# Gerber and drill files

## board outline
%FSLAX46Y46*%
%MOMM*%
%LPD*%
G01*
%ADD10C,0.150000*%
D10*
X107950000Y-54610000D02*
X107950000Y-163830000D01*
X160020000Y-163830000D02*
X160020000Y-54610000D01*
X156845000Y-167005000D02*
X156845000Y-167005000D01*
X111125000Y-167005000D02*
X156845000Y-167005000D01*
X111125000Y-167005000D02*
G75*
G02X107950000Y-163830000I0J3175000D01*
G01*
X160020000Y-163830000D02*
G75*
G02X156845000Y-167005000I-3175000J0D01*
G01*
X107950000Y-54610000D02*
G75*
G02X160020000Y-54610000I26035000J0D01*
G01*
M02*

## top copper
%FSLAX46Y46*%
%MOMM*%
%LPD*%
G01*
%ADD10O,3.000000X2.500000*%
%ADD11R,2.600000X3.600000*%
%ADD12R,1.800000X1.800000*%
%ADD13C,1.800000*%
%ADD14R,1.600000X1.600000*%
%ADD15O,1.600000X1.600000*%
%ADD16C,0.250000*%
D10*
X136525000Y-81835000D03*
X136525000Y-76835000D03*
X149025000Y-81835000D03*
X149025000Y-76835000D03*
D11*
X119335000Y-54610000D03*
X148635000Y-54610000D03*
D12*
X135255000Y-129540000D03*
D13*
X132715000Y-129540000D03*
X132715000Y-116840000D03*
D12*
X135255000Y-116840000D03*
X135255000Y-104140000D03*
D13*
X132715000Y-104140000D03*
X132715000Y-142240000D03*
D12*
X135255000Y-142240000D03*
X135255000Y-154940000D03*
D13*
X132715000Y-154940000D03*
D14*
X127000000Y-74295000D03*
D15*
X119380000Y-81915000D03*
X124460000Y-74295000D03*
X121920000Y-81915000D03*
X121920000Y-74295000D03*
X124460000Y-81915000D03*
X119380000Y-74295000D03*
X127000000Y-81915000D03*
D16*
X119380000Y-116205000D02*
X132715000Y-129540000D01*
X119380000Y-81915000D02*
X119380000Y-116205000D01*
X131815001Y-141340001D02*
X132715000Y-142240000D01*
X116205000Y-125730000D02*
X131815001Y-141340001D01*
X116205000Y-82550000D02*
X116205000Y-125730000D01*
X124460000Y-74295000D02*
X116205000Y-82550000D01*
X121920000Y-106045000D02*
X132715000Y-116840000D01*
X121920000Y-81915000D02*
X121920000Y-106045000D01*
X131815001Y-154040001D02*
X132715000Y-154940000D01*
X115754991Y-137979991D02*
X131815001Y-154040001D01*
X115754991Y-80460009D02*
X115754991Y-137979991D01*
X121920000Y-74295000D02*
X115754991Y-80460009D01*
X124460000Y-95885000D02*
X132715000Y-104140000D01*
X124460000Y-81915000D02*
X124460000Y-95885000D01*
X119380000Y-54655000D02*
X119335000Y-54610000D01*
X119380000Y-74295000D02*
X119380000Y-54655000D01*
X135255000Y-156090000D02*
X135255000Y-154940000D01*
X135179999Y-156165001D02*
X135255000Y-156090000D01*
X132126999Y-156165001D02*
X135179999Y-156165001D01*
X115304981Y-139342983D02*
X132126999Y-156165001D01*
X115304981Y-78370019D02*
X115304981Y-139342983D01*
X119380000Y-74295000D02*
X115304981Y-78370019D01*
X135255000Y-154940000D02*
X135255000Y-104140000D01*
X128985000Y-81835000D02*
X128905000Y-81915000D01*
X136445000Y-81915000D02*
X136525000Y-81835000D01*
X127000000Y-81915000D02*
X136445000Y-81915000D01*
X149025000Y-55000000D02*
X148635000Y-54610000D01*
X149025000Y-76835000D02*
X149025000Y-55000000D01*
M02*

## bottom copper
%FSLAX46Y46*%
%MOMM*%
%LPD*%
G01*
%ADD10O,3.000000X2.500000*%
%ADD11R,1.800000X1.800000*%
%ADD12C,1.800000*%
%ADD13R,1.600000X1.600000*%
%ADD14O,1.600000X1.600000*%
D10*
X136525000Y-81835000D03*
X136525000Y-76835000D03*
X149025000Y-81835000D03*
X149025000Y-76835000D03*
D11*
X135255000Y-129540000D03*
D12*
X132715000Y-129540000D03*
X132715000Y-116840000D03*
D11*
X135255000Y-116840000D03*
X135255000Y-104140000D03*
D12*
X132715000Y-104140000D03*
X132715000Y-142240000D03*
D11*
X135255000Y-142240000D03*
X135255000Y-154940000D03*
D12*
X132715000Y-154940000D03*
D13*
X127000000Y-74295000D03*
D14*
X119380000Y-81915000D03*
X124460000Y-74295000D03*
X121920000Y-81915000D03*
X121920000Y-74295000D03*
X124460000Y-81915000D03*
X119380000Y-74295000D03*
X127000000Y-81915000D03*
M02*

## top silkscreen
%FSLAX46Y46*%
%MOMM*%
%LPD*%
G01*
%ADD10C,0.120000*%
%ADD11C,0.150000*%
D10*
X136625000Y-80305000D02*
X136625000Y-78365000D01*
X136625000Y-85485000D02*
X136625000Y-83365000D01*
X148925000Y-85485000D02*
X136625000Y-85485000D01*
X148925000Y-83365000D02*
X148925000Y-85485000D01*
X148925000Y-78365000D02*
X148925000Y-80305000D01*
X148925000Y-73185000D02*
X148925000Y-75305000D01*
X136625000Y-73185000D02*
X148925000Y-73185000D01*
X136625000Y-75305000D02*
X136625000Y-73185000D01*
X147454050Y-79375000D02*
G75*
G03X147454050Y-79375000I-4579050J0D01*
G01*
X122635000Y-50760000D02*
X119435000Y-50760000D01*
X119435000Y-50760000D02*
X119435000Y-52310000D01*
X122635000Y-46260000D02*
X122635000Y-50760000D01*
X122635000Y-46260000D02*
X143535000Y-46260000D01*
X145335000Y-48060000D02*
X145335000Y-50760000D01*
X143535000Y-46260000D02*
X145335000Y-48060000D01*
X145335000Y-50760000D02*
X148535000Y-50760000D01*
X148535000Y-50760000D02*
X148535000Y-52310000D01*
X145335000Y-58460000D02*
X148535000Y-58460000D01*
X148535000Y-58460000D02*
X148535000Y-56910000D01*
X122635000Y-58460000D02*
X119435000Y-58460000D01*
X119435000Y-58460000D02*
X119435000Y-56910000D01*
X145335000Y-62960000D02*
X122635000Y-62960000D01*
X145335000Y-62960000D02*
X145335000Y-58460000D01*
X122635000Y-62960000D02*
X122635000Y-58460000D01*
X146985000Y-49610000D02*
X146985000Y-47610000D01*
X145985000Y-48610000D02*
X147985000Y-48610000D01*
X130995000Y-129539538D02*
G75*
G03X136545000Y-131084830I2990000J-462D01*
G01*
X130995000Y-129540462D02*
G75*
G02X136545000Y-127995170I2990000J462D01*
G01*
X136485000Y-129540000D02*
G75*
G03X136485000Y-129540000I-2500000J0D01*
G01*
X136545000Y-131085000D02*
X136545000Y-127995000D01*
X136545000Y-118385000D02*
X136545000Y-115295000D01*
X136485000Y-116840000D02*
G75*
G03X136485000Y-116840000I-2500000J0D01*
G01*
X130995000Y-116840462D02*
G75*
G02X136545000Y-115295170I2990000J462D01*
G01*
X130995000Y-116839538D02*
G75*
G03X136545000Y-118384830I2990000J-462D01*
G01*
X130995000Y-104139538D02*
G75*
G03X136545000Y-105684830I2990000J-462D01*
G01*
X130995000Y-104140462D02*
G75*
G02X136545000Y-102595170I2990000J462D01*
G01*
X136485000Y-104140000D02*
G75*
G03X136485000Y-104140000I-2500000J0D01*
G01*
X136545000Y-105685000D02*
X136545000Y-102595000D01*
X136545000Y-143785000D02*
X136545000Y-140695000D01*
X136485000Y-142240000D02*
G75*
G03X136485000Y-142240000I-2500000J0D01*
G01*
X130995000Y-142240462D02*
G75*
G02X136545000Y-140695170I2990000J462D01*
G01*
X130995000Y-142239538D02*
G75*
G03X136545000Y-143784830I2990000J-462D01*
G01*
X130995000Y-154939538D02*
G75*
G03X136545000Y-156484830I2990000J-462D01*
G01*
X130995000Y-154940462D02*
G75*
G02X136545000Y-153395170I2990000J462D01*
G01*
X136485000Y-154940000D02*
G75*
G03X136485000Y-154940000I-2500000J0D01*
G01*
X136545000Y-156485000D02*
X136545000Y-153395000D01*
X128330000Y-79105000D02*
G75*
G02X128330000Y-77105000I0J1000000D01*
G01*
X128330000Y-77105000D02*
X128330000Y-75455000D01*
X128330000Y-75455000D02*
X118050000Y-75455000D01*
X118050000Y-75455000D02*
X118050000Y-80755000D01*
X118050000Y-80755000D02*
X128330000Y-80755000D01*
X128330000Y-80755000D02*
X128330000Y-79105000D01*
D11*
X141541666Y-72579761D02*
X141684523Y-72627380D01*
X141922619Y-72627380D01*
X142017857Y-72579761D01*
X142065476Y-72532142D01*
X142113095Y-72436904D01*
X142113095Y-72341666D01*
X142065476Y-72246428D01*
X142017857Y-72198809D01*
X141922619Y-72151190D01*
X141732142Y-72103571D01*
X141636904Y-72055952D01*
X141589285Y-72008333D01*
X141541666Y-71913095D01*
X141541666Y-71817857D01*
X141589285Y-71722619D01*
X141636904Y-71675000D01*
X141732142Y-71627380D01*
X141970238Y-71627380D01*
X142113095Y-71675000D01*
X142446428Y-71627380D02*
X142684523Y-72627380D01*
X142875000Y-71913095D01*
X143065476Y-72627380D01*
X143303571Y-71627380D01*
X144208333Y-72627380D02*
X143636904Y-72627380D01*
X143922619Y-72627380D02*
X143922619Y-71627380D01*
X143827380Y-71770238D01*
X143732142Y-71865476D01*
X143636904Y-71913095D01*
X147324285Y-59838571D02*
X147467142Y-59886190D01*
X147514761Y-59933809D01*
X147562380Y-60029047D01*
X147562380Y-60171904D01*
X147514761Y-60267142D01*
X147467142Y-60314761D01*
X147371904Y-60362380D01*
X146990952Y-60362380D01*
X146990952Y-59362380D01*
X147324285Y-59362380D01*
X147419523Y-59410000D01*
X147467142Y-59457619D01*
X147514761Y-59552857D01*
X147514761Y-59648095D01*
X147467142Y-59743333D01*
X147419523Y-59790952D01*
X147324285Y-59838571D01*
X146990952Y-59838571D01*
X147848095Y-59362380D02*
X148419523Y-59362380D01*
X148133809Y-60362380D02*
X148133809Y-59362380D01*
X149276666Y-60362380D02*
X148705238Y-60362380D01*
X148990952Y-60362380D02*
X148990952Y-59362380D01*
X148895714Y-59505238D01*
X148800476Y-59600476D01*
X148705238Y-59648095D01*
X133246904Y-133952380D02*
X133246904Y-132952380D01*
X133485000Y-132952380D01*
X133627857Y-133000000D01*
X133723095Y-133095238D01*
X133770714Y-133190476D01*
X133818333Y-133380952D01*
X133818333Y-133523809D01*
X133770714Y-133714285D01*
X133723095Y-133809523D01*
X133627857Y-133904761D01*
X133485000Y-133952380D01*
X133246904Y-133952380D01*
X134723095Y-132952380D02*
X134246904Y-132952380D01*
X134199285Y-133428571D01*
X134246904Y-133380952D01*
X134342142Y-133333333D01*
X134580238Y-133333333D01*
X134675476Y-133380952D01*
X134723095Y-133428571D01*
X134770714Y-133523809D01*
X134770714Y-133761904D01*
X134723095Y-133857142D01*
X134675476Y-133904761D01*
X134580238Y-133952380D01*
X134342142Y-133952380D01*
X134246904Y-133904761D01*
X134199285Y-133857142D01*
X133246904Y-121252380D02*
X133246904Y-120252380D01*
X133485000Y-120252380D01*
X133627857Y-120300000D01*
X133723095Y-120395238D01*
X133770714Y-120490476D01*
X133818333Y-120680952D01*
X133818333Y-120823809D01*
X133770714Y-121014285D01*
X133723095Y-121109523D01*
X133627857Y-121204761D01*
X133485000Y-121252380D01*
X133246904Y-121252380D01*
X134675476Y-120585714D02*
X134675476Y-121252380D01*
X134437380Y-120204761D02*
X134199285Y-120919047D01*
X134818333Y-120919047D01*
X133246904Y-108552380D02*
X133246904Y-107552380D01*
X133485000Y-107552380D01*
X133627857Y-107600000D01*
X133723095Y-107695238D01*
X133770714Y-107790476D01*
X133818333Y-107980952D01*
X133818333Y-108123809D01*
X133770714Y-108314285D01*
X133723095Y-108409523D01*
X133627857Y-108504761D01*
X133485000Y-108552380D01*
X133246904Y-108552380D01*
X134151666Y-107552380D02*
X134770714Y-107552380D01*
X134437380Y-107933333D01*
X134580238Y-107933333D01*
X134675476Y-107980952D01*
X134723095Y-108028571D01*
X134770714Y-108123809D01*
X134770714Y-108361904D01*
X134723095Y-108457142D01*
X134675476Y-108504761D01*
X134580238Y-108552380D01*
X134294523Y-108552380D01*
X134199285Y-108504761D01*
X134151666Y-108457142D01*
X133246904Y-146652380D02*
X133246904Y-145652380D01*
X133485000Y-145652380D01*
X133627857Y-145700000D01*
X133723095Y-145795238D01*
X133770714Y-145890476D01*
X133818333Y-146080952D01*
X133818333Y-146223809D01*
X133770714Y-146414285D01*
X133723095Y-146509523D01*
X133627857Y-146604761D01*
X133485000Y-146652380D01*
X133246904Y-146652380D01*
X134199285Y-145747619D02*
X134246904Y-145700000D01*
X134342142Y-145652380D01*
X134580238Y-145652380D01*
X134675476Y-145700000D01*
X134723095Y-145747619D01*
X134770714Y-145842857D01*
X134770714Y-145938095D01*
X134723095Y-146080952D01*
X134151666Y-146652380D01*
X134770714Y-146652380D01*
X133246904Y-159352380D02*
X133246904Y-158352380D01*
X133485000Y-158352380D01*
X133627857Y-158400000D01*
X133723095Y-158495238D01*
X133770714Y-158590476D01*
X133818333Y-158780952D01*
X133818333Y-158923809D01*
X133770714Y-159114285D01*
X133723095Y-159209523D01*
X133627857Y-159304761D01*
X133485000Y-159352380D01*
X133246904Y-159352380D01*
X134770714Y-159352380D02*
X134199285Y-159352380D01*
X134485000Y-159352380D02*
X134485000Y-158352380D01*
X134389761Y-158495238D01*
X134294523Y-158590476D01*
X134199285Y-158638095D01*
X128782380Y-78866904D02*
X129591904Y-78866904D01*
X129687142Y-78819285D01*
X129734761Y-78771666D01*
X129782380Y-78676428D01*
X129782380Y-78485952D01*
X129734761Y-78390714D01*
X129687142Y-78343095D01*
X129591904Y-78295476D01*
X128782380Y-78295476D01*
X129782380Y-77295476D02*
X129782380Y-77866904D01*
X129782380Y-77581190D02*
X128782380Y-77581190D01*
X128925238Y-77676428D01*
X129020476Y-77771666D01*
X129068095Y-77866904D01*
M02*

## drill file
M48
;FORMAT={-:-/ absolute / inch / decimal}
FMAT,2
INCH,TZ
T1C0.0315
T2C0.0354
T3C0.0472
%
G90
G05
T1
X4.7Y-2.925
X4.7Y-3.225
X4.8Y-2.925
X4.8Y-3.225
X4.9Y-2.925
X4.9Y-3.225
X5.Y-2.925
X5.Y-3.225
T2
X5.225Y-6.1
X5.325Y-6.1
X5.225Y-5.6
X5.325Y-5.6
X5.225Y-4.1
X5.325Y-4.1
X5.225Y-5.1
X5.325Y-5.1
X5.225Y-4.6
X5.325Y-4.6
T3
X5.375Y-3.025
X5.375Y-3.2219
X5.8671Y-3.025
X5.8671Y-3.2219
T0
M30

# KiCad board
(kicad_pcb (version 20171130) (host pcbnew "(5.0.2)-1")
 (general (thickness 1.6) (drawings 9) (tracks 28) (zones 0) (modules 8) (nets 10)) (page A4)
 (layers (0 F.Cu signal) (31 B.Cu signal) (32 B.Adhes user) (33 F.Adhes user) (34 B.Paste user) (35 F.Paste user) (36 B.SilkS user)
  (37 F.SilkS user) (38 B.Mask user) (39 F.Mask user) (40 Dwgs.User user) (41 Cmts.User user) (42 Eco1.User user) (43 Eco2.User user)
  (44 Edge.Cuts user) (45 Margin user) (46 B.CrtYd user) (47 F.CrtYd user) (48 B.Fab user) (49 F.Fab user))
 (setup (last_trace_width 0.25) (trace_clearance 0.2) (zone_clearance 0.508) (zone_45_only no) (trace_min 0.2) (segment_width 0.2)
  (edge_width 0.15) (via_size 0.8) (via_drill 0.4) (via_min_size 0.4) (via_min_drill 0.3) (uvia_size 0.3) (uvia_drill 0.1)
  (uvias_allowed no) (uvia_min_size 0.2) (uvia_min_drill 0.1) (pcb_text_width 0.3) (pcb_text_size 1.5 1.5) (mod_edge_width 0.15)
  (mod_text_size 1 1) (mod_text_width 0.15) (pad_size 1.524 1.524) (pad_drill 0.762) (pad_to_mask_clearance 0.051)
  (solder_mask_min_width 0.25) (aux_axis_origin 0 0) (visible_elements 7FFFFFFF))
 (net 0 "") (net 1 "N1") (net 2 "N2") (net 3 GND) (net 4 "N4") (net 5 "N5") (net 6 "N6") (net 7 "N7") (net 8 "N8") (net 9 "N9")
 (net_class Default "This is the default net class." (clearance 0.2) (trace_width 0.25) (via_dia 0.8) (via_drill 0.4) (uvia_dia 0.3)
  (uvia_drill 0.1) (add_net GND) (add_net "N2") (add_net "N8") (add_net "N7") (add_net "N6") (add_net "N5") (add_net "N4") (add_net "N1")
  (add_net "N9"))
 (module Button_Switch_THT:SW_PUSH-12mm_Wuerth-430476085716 (layer F.Cu) (at 136.525 76.835)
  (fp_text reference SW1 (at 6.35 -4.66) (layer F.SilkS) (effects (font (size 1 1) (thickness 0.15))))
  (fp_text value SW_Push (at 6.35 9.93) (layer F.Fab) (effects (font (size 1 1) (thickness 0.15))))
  (fp_line (start 0.1 3.47) (end 0.1 1.53) (layer F.SilkS) (width 0.12))
  (fp_line (start 0.1 8.65) (end 0.1 6.53) (layer F.SilkS) (width 0.12))
  (fp_line (start 12.4 8.65) (end 0.1 8.65) (layer F.SilkS) (width 0.12))
  (fp_line (start 12.4 6.53) (end 12.4 8.65) (layer F.SilkS) (width 0.12))
  (fp_line (start 12.4 1.53) (end 12.4 3.47) (layer F.SilkS) (width 0.12))
  (fp_line (start 12.4 -3.65) (end 12.4 -1.53) (layer F.SilkS) (width 0.12))
  (fp_line (start 0.1 -3.65) (end 12.4 -3.65) (layer F.SilkS) (width 0.12))
  (fp_line (start 0.1 -1.53) (end 0.1 -3.65) (layer F.SilkS) (width 0.12))
  (fp_circle (center 6.35 2.54) (end 10.92905 2.54) (layer F.SilkS) (width 0.12))
  (pad 2 thru_hole oval (at 0 5) (size 3 2.5) (drill 1.2) (layers *.Cu *.Mask) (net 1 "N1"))
  (pad 1 thru_hole oval (at 0 0) (size 3 2.5) (drill 1.2) (layers *.Cu *.Mask) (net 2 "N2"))
  (pad 2 thru_hole oval (at 12.5 5) (size 3 2.5) (drill 1.2) (layers *.Cu *.Mask) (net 1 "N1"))
  (pad 1 thru_hole oval (at 12.5 0) (size 3 2.5) (drill 1.2) (layers *.Cu *.Mask) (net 2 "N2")))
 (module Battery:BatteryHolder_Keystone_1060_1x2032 (layer F.Cu) (at 133.985 54.61 180)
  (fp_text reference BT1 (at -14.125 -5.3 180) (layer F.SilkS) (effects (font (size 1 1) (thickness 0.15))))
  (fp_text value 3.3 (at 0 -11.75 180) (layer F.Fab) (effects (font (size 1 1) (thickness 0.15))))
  (fp_line (start 11.35 3.85) (end 14.55 3.85) (layer F.SilkS) (width 0.12))
  (fp_line (start 14.55 3.85) (end 14.55 2.3) (layer F.SilkS) (width 0.12))
  (fp_line (start 11.35 8.35) (end 11.35 3.85) (layer F.SilkS) (width 0.12))
  (fp_line (start 11.35 8.35) (end -9.55 8.35) (layer F.SilkS) (width 0.12))
  (fp_line (start -11.35 6.55) (end -11.35 3.85) (layer F.SilkS) (width 0.12))
  (fp_line (start -9.55 8.35) (end -11.35 6.55) (layer F.SilkS) (width 0.12))
  (fp_line (start -11.35 3.85) (end -14.55 3.85) (layer F.SilkS) (width 0.12))
  (fp_line (start -14.55 3.85) (end -14.55 2.3) (layer F.SilkS) (width 0.12))
  (fp_line (start -11.35 -3.85) (end -14.55 -3.85) (layer F.SilkS) (width 0.12))
  (fp_line (start -14.55 -3.85) (end -14.55 -2.3) (layer F.SilkS) (width 0.12))
  (fp_line (start 11.35 -3.85) (end 14.55 -3.85) (layer F.SilkS) (width 0.12))
  (fp_line (start 14.55 -3.85) (end 14.55 -2.3) (layer F.SilkS) (width 0.12))
  (fp_line (start -11.35 -8.35) (end 11.35 -8.35) (layer F.SilkS) (width 0.12))
  (fp_line (start -11.35 -8.35) (end -11.35 -3.85) (layer F.SilkS) (width 0.12))
  (fp_line (start 11.35 -8.35) (end 11.35 -3.85) (layer F.SilkS) (width 0.12))
  (fp_line (start -13 5) (end -13 7) (layer F.SilkS) (width 0.12))
  (fp_line (start -12 6) (end -14 6) (layer F.SilkS) (width 0.12))
  (pad 2 smd rect (at 14.65 0) (size 2.6 3.6) (layers F.Cu F.Paste F.Mask) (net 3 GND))
  (pad 1 smd rect (at -14.65 0) (size 2.6 3.6) (layers F.Cu F.Paste F.Mask) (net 2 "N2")))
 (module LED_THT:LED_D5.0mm (layer F.Cu) (at 135.255 129.54 180)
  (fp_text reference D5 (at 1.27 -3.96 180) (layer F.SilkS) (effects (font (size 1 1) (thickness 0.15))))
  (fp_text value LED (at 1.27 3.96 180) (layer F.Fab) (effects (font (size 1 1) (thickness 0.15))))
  (fp_arc (start 1.27 0) (end -1.29 -1.54483) (angle 148.9) (layer F.SilkS) (width 0.12))
  (fp_arc (start 1.27 0) (end -1.29 1.54483) (angle -148.9) (layer F.SilkS) (width 0.12))
  (fp_circle (center 1.27 0) (end 3.77 0) (layer F.SilkS) (width 0.12))
  (fp_line (start -1.29 -1.545) (end -1.29 1.545) (layer F.SilkS) (width 0.12))
  (pad 1 thru_hole rect (at 0 0 180) (size 1.8 1.8) (drill 0.9) (layers *.Cu *.Mask) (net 3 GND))
  (pad 2 thru_hole circle (at 2.54 0 180) (size 1.8 1.8) (drill 0.9) (layers *.Cu *.Mask) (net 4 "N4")))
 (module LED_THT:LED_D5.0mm (layer F.Cu) (at 135.255 116.84 180)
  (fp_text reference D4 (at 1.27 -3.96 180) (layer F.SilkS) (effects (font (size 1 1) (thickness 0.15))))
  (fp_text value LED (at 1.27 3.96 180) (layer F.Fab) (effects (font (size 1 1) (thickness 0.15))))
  (fp_line (start -1.29 -1.545) (end -1.29 1.545) (layer F.SilkS) (width 0.12))
  (fp_circle (center 1.27 0) (end 3.77 0) (layer F.SilkS) (width 0.12))
  (fp_arc (start 1.27 0) (end -1.29 1.54483) (angle -148.9) (layer F.SilkS) (width 0.12))
  (fp_arc (start 1.27 0) (end -1.29 -1.54483) (angle 148.9) (layer F.SilkS) (width 0.12))
  (pad 2 thru_hole circle (at 2.54 0 180) (size 1.8 1.8) (drill 0.9) (layers *.Cu *.Mask) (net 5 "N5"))
  (pad 1 thru_hole rect (at 0 0 180) (size 1.8 1.8) (drill 0.9) (layers *.Cu *.Mask) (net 3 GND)))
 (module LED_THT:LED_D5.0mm (layer F.Cu) (at 135.255 104.14 180)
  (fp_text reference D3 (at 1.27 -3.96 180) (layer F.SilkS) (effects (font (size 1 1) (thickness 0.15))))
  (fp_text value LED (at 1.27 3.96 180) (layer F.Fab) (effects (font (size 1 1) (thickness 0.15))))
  (fp_arc (start 1.27 0) (end -1.29 -1.54483) (angle 148.9) (layer F.SilkS) (width 0.12))
  (fp_arc (start 1.27 0) (end -1.29 1.54483) (angle -148.9) (layer F.SilkS) (width 0.12))
  (fp_circle (center 1.27 0) (end 3.77 0) (layer F.SilkS) (width 0.12))
  (fp_line (start -1.29 -1.545) (end -1.29 1.545) (layer F.SilkS) (width 0.12))
  (pad 1 thru_hole rect (at 0 0 180) (size 1.8 1.8) (drill 0.9) (layers *.Cu *.Mask) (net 3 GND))
  (pad 2 thru_hole circle (at 2.54 0 180) (size 1.8 1.8) (drill 0.9) (layers *.Cu *.Mask) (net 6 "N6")))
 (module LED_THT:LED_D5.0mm (layer F.Cu) (at 135.255 142.24 180)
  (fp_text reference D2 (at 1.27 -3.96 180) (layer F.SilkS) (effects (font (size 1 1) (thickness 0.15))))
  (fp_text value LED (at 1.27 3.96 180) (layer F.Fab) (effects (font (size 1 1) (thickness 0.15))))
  (fp_line (start -1.29 -1.545) (end -1.29 1.545) (layer F.SilkS) (width 0.12))
  (fp_circle (center 1.27 0) (end 3.77 0) (layer F.SilkS) (width 0.12))
  (fp_arc (start 1.27 0) (end -1.29 1.54483) (angle -148.9) (layer F.SilkS) (width 0.12))
  (fp_arc (start 1.27 0) (end -1.29 -1.54483) (angle 148.9) (layer F.SilkS) (width 0.12))
  (pad 2 thru_hole circle (at 2.54 0 180) (size 1.8 1.8) (drill 0.9) (layers *.Cu *.Mask) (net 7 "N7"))
  (pad 1 thru_hole rect (at 0 0 180) (size 1.8 1.8) (drill 0.9) (layers *.Cu *.Mask) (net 3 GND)))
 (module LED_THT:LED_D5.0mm (layer F.Cu) (at 135.255 154.94 180)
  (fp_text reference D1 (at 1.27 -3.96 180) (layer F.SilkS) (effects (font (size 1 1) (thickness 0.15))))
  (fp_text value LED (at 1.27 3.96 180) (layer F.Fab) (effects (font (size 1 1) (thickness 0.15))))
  (fp_arc (start 1.27 0) (end -1.29 -1.54483) (angle 148.9) (layer F.SilkS) (width 0.12))
  (fp_arc (start 1.27 0) (end -1.29 1.54483) (angle -148.9) (layer F.SilkS) (width 0.12))
  (fp_circle (center 1.27 0) (end 3.77 0) (layer F.SilkS) (width 0.12))
  (fp_line (start -1.29 -1.545) (end -1.29 1.545) (layer F.SilkS) (width 0.12))
  (pad 1 thru_hole rect (at 0 0 180) (size 1.8 1.8) (drill 0.9) (layers *.Cu *.Mask) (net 3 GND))
  (pad 2 thru_hole circle (at 2.54 0 180) (size 1.8 1.8) (drill 0.9) (layers *.Cu *.Mask) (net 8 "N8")))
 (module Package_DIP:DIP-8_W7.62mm (layer F.Cu) (at 127 74.295 270)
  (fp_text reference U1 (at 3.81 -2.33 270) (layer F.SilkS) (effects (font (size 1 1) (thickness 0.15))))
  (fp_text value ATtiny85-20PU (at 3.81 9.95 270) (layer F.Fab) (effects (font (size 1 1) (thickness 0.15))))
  (fp_arc (start 3.81 -1.33) (end 2.81 -1.33) (angle -180) (layer F.SilkS) (width 0.12))
  (fp_line (start 2.81 -1.33) (end 1.16 -1.33) (layer F.SilkS) (width 0.12))
  (fp_line (start 1.16 -1.33) (end 1.16 8.95) (layer F.SilkS) (width 0.12))
  (fp_line (start 1.16 8.95) (end 6.46 8.95) (layer F.SilkS) (width 0.12))
  (fp_line (start 6.46 8.95) (end 6.46 -1.33) (layer F.SilkS) (width 0.12))
  (fp_line (start 6.46 -1.33) (end 4.81 -1.33) (layer F.SilkS) (width 0.12))
  (pad 1 thru_hole rect (at 0 0 270) (size 1.6 1.6) (drill 0.8) (layers *.Cu *.Mask) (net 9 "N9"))
  (pad 5 thru_hole oval (at 7.62 7.62 270) (size 1.6 1.6) (drill 0.8) (layers *.Cu *.Mask) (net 4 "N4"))
  (pad 2 thru_hole oval (at 0 2.54 270) (size 1.6 1.6) (drill 0.8) (layers *.Cu *.Mask) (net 7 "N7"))
  (pad 6 thru_hole oval (at 7.62 5.08 270) (size 1.6 1.6) (drill 0.8) (layers *.Cu *.Mask) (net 5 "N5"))
  (pad 3 thru_hole oval (at 0 5.08 270) (size 1.6 1.6) (drill 0.8) (layers *.Cu *.Mask) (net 8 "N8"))
  (pad 7 thru_hole oval (at 7.62 2.54 270) (size 1.6 1.6) (drill 0.8) (layers *.Cu *.Mask) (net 6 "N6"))
  (pad 4 thru_hole oval (at 0 7.62 270) (size 1.6 1.6) (drill 0.8) (layers *.Cu *.Mask) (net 3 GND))
  (pad 8 thru_hole oval (at 7.62 0 270) (size 1.6 1.6) (drill 0.8) (layers *.Cu *.Mask) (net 1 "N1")))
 (gr_line (start 107.95 54.61) (end 107.95 163.83) (layer Edge.Cuts) (width 0.15))
 (gr_line (start 160.02 163.83) (end 160.02 54.61) (layer Edge.Cuts) (width 0.15))
 (gr_line (start 156.845 167.005) (end 156.845 167.005) (layer Edge.Cuts) (width 0.15))
 (gr_line (start 111.125 167.005) (end 156.845 167.005) (layer Edge.Cuts) (width 0.15))
 (gr_arc (start 111.125 163.83) (end 107.95 163.83) (angle -90) (layer Edge.Cuts) (width 0.15))
 (gr_arc (start 156.845 163.83) (end 156.845 167.005) (angle -90) (layer Edge.Cuts) (width 0.15))
 (gr_arc (start 133.985 54.61) (end 160.02 54.61) (angle -180) (layer Edge.Cuts) (width 0.15))
 (segment (start 119.38 116.205) (end 132.715 129.54) (width 0.25) (layer F.Cu) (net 4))
 (segment (start 119.38 81.915) (end 119.38 116.205) (width 0.25) (layer F.Cu) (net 4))
 (segment (start 131.815001 141.340001) (end 132.715 142.24) (width 0.25) (layer F.Cu) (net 7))
 (segment (start 116.205 125.73) (end 131.815001 141.340001) (width 0.25) (layer F.Cu) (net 7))
 (segment (start 116.205 82.55) (end 116.205 125.73) (width 0.25) (layer F.Cu) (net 7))
 (segment (start 124.46 74.295) (end 116.205 82.55) (width 0.25) (layer F.Cu) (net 7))
 (segment (start 121.92 106.045) (end 132.715 116.84) (width 0.25) (layer F.Cu) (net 5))
 (segment (start 121.92 81.915) (end 121.92 106.045) (width 0.25) (layer F.Cu) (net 5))
 (segment (start 131.815001 154.040001) (end 132.715 154.94) (width 0.25) (layer F.Cu) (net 8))
 (segment (start 115.754991 137.979991) (end 131.815001 154.040001) (width 0.25) (layer F.Cu) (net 8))
 (segment (start 115.754991 80.460009) (end 115.754991 137.979991) (width 0.25) (layer F.Cu) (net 8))
 (segment (start 121.92 74.295) (end 115.754991 80.460009) (width 0.25) (layer F.Cu) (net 8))
 (segment (start 124.46 95.885) (end 132.715 104.14) (width 0.25) (layer F.Cu) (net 6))
 (segment (start 124.46 81.915) (end 124.46 95.885) (width 0.25) (layer F.Cu) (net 6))
 (segment (start 119.38 54.655) (end 119.335 54.61) (width 0.25) (layer F.Cu) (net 3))
 (segment (start 119.38 74.295) (end 119.38 54.655) (width 0.25) (layer F.Cu) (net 3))
 (segment (start 135.255 156.09) (end 135.255 154.94) (width 0.25) (layer F.Cu) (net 3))
 (segment (start 135.179999 156.165001) (end 135.255 156.09) (width 0.25) (layer F.Cu) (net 3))
 (segment (start 132.126999 156.165001) (end 135.179999 156.165001) (width 0.25) (layer F.Cu) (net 3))
 (segment (start 115.304981 139.342983) (end 132.126999 156.165001) (width 0.25) (layer F.Cu) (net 3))
 (segment (start 115.304981 78.370019) (end 115.304981 139.342983) (width 0.25) (layer F.Cu) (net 3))
 (segment (start 119.38 74.295) (end 115.304981 78.370019) (width 0.25) (layer F.Cu) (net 3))
 (segment (start 135.255 154.94) (end 135.255 104.14) (width 0.25) (layer F.Cu) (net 3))
 (segment (start 128.985 81.835) (end 128.905 81.915) (width 0.25) (layer F.Cu) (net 1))
 (segment (start 136.445 81.915) (end 136.525 81.835) (width 0.25) (layer F.Cu) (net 1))
 (segment (start 127 81.915) (end 136.445 81.915) (width 0.25) (layer F.Cu) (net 1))
 (segment (start 149.025 55) (end 148.635 54.61) (width 0.25) (layer F.Cu) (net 2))
 (segment (start 149.025 76.835) (end 149.025 55) (width 0.25) (layer F.Cu) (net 2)))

